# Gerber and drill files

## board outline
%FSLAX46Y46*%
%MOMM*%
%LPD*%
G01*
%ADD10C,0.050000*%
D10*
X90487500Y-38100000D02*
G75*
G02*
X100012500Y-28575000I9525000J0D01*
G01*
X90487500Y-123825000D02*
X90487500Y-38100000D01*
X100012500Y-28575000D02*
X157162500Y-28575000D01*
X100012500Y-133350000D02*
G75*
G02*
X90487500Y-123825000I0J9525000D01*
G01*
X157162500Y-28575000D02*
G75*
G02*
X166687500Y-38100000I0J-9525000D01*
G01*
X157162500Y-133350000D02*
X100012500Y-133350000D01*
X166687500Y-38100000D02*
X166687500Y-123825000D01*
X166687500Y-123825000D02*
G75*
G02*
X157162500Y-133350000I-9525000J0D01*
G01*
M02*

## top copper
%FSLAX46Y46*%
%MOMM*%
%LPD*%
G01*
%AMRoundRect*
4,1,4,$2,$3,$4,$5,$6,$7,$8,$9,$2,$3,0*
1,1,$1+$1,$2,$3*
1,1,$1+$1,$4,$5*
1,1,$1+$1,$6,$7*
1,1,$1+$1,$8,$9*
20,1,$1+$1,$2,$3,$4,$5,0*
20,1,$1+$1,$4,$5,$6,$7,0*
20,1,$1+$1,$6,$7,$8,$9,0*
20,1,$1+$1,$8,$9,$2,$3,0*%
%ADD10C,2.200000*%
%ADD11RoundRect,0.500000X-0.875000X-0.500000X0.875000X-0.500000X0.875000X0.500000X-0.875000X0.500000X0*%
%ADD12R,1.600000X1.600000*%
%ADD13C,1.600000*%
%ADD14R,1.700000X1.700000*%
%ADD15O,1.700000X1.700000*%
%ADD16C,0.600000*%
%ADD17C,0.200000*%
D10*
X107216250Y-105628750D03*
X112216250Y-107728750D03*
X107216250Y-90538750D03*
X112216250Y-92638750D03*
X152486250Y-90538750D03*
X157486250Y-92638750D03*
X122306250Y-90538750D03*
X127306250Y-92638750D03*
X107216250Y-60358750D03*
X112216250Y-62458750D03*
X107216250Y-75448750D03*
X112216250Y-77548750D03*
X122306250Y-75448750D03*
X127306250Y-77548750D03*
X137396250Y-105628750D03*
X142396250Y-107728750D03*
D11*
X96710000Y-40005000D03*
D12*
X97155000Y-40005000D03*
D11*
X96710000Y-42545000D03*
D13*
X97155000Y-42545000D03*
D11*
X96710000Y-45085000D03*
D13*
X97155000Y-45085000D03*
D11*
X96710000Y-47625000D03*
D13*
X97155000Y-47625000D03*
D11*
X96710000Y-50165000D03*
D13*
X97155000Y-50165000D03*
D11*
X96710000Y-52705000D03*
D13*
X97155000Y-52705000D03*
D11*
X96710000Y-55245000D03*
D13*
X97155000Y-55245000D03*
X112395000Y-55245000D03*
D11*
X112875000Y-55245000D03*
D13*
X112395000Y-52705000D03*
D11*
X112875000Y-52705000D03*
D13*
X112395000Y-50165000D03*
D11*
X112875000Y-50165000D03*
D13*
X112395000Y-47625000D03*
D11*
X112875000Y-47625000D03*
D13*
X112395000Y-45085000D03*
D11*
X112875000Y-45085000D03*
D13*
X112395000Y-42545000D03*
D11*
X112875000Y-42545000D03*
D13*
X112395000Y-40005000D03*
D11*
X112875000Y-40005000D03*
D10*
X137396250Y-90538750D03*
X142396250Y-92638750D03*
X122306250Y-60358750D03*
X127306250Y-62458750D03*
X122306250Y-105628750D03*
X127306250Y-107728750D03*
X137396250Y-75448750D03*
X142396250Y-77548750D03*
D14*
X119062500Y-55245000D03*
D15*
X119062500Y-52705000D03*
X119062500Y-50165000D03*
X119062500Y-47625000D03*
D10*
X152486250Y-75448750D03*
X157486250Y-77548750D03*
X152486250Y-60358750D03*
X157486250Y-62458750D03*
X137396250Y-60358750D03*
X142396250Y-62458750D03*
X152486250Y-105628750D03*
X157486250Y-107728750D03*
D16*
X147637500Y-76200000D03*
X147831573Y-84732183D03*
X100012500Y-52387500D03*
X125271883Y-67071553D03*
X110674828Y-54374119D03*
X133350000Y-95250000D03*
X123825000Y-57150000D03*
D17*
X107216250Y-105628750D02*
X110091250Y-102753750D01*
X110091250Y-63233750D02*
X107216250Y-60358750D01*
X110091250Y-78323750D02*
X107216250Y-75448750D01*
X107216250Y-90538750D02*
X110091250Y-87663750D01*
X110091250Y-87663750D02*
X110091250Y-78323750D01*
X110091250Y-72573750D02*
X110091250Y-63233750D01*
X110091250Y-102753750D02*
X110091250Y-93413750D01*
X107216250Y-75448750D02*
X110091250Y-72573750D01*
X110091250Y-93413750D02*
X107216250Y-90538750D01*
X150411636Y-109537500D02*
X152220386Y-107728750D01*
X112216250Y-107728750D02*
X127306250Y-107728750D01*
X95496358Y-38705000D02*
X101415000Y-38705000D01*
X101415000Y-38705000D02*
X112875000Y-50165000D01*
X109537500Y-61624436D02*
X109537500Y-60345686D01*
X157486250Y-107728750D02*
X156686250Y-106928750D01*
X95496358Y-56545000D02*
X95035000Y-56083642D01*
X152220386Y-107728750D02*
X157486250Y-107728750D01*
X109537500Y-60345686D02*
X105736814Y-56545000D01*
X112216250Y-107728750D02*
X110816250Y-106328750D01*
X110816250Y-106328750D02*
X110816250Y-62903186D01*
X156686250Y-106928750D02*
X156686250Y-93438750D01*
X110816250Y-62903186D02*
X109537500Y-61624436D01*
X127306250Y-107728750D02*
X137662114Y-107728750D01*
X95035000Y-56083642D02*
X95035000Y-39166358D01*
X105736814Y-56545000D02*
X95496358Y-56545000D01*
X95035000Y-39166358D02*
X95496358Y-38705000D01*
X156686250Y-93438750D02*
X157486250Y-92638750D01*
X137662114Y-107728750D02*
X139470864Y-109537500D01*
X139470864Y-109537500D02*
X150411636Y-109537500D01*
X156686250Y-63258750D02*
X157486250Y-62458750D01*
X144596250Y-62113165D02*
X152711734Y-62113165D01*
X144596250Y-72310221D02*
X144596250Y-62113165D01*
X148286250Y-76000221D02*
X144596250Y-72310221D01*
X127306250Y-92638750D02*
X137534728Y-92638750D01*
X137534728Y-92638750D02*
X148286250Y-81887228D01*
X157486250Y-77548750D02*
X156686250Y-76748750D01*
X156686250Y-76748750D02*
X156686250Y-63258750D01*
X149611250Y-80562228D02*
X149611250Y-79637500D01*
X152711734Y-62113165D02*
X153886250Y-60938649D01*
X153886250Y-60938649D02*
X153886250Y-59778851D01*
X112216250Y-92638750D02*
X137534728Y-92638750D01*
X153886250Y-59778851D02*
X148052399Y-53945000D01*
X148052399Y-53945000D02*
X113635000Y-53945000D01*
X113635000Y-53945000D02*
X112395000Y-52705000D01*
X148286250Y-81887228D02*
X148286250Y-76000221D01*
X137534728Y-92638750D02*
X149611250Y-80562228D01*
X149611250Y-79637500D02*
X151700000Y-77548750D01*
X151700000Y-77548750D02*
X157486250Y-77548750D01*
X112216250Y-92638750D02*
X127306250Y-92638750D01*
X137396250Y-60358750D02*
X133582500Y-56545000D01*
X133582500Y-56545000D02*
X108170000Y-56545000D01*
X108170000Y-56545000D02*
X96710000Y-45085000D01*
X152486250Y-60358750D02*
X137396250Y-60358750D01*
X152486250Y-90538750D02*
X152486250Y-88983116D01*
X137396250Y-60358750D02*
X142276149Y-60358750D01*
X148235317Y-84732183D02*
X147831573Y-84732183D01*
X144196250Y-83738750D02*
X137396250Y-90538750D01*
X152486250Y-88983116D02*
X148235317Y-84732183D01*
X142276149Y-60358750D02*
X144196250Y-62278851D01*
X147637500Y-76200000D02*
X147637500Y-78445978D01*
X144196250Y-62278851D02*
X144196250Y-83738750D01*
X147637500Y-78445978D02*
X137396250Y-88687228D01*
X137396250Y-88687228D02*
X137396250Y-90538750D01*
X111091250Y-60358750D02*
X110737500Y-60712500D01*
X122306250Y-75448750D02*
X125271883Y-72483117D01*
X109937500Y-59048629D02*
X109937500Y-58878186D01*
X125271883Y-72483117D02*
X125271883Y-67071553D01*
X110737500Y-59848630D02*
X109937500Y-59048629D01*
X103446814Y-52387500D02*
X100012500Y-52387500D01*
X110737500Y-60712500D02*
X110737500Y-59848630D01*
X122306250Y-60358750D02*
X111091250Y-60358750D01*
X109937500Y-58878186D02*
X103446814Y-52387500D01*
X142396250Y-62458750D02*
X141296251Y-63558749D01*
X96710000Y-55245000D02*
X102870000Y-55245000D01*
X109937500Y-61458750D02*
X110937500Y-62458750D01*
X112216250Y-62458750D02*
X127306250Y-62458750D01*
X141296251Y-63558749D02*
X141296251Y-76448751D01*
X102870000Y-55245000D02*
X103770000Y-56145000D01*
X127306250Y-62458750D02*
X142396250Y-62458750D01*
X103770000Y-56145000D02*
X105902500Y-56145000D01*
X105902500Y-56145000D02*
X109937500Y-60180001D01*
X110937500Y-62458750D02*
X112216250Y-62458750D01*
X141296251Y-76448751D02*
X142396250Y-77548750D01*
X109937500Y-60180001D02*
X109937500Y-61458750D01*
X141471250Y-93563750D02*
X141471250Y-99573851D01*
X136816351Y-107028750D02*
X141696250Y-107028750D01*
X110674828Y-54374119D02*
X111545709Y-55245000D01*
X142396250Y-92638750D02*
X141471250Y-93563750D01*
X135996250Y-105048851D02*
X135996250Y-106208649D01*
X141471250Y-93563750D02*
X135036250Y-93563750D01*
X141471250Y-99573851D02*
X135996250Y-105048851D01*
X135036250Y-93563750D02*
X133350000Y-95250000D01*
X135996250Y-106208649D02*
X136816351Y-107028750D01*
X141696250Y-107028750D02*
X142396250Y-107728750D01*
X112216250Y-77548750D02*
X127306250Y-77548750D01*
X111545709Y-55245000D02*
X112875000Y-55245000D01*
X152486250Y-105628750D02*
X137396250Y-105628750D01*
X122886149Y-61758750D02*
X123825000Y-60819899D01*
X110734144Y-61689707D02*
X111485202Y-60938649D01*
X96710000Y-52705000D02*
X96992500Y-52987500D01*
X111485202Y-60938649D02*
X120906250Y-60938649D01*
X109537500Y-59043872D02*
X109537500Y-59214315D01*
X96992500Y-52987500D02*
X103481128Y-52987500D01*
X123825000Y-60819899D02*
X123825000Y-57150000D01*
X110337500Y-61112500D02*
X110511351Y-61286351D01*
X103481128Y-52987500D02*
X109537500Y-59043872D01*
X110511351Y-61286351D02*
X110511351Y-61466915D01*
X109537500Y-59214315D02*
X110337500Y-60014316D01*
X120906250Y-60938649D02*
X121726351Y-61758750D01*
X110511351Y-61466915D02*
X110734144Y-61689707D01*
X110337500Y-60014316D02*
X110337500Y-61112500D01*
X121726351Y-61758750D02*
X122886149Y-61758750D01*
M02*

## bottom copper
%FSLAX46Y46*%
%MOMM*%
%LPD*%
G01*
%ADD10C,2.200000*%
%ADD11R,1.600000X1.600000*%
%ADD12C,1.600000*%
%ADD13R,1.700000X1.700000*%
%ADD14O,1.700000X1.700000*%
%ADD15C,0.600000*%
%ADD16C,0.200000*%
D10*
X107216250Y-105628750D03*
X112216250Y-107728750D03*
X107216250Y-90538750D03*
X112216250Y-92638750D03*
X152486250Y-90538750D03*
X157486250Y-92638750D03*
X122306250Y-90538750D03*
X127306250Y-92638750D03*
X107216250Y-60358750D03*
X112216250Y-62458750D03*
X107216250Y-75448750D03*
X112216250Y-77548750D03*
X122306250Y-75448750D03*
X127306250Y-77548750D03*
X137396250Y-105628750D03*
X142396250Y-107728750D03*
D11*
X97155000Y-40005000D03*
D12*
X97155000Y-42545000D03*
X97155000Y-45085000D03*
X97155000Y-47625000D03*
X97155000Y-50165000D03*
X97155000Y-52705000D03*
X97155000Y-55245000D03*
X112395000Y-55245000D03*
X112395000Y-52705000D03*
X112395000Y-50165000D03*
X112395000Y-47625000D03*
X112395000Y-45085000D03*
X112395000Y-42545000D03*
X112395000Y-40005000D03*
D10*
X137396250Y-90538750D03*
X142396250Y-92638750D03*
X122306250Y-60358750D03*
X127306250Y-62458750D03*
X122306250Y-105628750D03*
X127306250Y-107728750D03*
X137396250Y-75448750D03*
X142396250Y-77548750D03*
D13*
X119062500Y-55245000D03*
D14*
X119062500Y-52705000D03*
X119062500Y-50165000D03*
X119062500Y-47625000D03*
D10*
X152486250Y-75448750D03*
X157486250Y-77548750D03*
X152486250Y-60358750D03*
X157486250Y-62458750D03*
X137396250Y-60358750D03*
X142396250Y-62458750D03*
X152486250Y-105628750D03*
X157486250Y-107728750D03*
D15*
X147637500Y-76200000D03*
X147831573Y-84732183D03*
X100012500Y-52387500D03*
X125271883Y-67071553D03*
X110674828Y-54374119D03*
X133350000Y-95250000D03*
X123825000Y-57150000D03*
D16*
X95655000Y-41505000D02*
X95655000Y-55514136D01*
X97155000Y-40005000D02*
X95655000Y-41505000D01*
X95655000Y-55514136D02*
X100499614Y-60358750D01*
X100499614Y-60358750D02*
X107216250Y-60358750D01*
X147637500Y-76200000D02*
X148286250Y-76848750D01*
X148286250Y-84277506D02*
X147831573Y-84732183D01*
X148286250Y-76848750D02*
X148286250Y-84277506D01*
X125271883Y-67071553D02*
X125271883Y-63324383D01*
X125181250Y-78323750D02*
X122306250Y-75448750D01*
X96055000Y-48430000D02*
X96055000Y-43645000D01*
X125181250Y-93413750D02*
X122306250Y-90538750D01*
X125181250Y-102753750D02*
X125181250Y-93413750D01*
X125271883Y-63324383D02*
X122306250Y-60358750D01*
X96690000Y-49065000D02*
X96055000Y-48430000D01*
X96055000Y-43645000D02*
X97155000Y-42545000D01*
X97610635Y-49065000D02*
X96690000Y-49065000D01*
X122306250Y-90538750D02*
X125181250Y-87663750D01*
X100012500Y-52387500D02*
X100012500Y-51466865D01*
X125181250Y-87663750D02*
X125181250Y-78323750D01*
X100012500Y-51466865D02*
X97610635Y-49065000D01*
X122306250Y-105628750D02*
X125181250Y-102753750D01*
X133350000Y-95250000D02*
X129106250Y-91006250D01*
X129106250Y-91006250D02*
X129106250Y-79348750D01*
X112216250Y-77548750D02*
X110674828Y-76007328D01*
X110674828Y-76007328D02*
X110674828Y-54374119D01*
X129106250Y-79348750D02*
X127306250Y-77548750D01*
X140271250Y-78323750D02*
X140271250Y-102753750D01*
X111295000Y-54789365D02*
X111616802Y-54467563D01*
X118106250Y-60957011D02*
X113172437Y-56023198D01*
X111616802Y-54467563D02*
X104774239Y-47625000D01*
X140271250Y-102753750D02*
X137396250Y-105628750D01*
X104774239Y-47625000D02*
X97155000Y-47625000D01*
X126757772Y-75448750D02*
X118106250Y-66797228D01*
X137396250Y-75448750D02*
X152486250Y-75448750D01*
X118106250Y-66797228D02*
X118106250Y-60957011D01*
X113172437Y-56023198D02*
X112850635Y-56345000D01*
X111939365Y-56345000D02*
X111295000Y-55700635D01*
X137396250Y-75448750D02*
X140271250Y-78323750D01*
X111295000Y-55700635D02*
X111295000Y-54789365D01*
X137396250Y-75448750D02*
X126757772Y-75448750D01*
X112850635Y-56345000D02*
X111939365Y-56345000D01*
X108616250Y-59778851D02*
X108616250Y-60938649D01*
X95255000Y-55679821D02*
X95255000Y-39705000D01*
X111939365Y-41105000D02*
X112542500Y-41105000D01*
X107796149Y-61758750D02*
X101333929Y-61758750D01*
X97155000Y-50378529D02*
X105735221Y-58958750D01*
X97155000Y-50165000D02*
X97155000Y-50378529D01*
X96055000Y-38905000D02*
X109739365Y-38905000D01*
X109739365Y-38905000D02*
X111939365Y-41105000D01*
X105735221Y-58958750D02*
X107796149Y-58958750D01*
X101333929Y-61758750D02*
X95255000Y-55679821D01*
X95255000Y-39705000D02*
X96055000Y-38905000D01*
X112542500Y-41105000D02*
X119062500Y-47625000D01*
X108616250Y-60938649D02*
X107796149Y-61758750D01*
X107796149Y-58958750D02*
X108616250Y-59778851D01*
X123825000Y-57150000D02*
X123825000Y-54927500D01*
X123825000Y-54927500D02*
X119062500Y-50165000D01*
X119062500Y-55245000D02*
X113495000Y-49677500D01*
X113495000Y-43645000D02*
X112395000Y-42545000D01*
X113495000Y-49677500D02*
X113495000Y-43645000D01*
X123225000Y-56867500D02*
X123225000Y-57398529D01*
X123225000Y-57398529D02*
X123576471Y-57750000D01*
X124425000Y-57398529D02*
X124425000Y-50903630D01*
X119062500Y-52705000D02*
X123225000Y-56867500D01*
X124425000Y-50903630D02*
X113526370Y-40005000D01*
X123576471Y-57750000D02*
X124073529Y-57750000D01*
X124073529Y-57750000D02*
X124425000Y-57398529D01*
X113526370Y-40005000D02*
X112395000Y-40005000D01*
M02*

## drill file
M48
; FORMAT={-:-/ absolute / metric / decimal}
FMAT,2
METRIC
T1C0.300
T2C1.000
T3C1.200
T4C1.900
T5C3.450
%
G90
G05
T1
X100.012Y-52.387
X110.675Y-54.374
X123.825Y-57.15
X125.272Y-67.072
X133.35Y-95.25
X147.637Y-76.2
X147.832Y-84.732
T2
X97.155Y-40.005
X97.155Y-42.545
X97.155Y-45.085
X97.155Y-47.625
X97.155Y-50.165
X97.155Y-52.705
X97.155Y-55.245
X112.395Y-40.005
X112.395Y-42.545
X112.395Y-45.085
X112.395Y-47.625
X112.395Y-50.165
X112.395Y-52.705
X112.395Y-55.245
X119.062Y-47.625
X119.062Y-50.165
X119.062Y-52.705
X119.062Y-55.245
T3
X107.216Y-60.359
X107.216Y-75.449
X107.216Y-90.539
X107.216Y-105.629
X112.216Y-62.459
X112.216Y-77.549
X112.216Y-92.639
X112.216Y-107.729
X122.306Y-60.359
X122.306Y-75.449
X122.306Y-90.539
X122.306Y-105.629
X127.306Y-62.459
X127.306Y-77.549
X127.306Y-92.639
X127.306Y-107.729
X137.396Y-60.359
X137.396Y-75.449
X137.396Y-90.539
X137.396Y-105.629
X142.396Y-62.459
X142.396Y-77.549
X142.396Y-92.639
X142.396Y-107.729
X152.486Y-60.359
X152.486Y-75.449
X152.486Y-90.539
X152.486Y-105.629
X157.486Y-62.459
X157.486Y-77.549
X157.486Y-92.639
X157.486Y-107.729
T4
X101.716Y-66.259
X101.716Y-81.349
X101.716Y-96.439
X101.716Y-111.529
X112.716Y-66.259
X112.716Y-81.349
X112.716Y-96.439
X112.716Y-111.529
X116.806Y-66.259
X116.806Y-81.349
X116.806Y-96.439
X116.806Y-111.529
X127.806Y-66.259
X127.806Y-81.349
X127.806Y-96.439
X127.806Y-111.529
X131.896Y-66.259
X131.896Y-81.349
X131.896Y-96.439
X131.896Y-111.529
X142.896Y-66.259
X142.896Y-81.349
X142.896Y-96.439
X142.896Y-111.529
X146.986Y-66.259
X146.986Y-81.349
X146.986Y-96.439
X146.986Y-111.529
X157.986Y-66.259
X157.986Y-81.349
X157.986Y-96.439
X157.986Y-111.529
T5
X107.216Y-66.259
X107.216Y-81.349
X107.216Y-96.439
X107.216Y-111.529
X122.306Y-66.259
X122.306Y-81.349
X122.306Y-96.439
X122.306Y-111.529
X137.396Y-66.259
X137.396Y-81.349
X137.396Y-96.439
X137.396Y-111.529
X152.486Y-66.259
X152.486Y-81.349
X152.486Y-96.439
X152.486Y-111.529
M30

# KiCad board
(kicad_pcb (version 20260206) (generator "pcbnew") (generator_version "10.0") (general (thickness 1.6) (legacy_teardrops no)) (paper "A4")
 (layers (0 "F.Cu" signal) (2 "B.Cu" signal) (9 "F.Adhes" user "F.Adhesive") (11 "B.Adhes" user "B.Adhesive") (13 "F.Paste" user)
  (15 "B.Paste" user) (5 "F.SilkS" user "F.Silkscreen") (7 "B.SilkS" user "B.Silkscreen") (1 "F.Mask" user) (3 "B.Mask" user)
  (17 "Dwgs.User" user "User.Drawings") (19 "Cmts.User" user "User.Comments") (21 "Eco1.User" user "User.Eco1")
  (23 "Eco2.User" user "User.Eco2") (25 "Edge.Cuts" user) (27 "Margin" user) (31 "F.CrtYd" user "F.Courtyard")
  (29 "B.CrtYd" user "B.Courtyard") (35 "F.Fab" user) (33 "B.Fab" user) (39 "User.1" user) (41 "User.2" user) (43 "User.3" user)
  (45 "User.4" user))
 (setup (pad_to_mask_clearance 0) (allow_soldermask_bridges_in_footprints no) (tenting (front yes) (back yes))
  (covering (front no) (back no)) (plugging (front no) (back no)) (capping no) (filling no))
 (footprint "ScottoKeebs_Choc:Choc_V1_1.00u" (layer "F.Cu") (at 107.21625 111.52875)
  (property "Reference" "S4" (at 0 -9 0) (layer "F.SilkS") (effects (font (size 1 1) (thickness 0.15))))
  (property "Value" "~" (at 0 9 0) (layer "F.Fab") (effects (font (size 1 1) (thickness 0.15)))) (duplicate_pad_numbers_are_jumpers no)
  (pad "" np_thru_hole circle (at -5.5 0) (size 1.9 1.9) (drill 1.9) (layers "*.Cu" "*.Mask"))
  (pad "" np_thru_hole circle (at 0 0) (size 3.45 3.45) (drill 3.45) (layers "*.Cu" "*.Mask"))
  (pad "" np_thru_hole circle (at 5.5 0) (size 1.9 1.9) (drill 1.9) (layers "*.Cu" "*.Mask"))
  (pad "1" thru_hole circle (at 0 -5.9) (size 2.2 2.2) (drill 1.2) (layers "*.Cu" "*.Mask") (remove_unused_layers no) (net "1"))
  (pad "2" thru_hole circle (at 5 -3.8) (size 2.2 2.2) (drill 1.2) (layers "*.Cu" "*.Mask") (remove_unused_layers no) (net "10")))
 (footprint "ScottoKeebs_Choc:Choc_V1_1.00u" (layer "F.Cu") (at 107.21625 96.43875)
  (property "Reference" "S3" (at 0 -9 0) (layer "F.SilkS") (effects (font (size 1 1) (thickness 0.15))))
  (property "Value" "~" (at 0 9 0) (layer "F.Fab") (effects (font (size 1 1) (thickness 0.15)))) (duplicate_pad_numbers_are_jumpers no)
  (pad "" np_thru_hole circle (at -5.5 0) (size 1.9 1.9) (drill 1.9) (layers "*.Cu" "*.Mask"))
  (pad "" np_thru_hole circle (at 0 0) (size 3.45 3.45) (drill 3.45) (layers "*.Cu" "*.Mask"))
  (pad "" np_thru_hole circle (at 5.5 0) (size 1.9 1.9) (drill 1.9) (layers "*.Cu" "*.Mask"))
  (pad "1" thru_hole circle (at 0 -5.9) (size 2.2 2.2) (drill 1.2) (layers "*.Cu" "*.Mask") (remove_unused_layers no) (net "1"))
  (pad "2" thru_hole circle (at 5 -3.8) (size 2.2 2.2) (drill 1.2) (layers "*.Cu" "*.Mask") (remove_unused_layers no) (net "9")))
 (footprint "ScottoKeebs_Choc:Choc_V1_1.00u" (layer "F.Cu") (at 152.48625 96.43875)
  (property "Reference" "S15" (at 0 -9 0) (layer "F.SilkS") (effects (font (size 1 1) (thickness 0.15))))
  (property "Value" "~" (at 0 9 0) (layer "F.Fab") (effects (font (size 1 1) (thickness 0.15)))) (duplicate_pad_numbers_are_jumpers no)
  (pad "" np_thru_hole circle (at -5.5 0) (size 1.9 1.9) (drill 1.9) (layers "*.Cu" "*.Mask"))
  (pad "" np_thru_hole circle (at 0 0) (size 3.45 3.45) (drill 3.45) (layers "*.Cu" "*.Mask"))
  (pad "" np_thru_hole circle (at 5.5 0) (size 1.9 1.9) (drill 1.9) (layers "*.Cu" "*.Mask"))
  (pad "1" thru_hole circle (at 0 -5.9) (size 2.2 2.2) (drill 1.2) (layers "*.Cu" "*.Mask") (remove_unused_layers no) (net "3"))
  (pad "2" thru_hole circle (at 5 -3.8) (size 2.2 2.2) (drill 1.2) (layers "*.Cu" "*.Mask") (remove_unused_layers no) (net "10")))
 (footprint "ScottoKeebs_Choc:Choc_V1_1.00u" (layer "F.Cu") (at 122.30625 96.43875)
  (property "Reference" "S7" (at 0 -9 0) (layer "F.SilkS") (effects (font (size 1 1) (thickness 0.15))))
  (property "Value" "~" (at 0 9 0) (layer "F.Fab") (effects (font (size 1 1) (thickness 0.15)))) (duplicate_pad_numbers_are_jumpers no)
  (pad "" np_thru_hole circle (at -5.5 0) (size 1.9 1.9) (drill 1.9) (layers "*.Cu" "*.Mask"))
  (pad "" np_thru_hole circle (at 0 0) (size 3.45 3.45) (drill 3.45) (layers "*.Cu" "*.Mask"))
  (pad "" np_thru_hole circle (at 5.5 0) (size 1.9 1.9) (drill 1.9) (layers "*.Cu" "*.Mask"))
  (pad "1" thru_hole circle (at 0 -5.9) (size 2.2 2.2) (drill 1.2) (layers "*.Cu" "*.Mask") (remove_unused_layers no) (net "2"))
  (pad "2" thru_hole circle (at 5 -3.8) (size 2.2 2.2) (drill 1.2) (layers "*.Cu" "*.Mask") (remove_unused_layers no) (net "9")))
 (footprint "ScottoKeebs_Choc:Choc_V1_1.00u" (layer "F.Cu") (at 107.21625 66.25875)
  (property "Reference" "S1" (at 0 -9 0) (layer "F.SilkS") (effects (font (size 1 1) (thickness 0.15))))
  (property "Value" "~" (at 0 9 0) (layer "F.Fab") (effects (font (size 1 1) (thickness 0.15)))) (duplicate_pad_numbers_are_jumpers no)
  (pad "" np_thru_hole circle (at -5.5 0) (size 1.9 1.9) (drill 1.9) (layers "*.Cu" "*.Mask"))
  (pad "" np_thru_hole circle (at 0 0) (size 3.45 3.45) (drill 3.45) (layers "*.Cu" "*.Mask"))
  (pad "" np_thru_hole circle (at 5.5 0) (size 1.9 1.9) (drill 1.9) (layers "*.Cu" "*.Mask"))
  (pad "1" thru_hole circle (at 0 -5.9) (size 2.2 2.2) (drill 1.2) (layers "*.Cu" "*.Mask") (remove_unused_layers no) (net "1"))
  (pad "2" thru_hole circle (at 5 -3.8) (size 2.2 2.2) (drill 1.2) (layers "*.Cu" "*.Mask") (remove_unused_layers no) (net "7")))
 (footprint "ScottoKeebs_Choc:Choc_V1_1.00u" (layer "F.Cu") (at 107.21625 81.34875)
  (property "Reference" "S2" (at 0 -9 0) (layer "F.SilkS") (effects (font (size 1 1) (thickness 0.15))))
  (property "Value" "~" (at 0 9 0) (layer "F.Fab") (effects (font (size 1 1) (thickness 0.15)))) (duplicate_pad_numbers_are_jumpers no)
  (pad "" np_thru_hole circle (at -5.5 0) (size 1.9 1.9) (drill 1.9) (layers "*.Cu" "*.Mask"))
  (pad "" np_thru_hole circle (at 0 0) (size 3.45 3.45) (drill 3.45) (layers "*.Cu" "*.Mask"))
  (pad "" np_thru_hole circle (at 5.5 0) (size 1.9 1.9) (drill 1.9) (layers "*.Cu" "*.Mask"))
  (pad "1" thru_hole circle (at 0 -5.9) (size 2.2 2.2) (drill 1.2) (layers "*.Cu" "*.Mask") (remove_unused_layers no) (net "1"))
  (pad "2" thru_hole circle (at 5 -3.8) (size 2.2 2.2) (drill 1.2) (layers "*.Cu" "*.Mask") (remove_unused_layers no) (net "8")))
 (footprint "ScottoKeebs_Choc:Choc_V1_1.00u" (layer "F.Cu") (at 122.30625 81.34875)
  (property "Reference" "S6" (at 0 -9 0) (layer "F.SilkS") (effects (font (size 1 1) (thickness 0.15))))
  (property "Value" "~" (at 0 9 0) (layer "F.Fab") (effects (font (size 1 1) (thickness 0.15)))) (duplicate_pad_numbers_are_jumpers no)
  (pad "" np_thru_hole circle (at -5.5 0) (size 1.9 1.9) (drill 1.9) (layers "*.Cu" "*.Mask"))
  (pad "" np_thru_hole circle (at 0 0) (size 3.45 3.45) (drill 3.45) (layers "*.Cu" "*.Mask"))
  (pad "" np_thru_hole circle (at 5.5 0) (size 1.9 1.9) (drill 1.9) (layers "*.Cu" "*.Mask"))
  (pad "1" thru_hole circle (at 0 -5.9) (size 2.2 2.2) (drill 1.2) (layers "*.Cu" "*.Mask") (remove_unused_layers no) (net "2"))
  (pad "2" thru_hole circle (at 5 -3.8) (size 2.2 2.2) (drill 1.2) (layers "*.Cu" "*.Mask") (remove_unused_layers no) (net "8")))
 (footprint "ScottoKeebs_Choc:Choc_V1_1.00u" (layer "F.Cu") (at 137.39625 111.52875)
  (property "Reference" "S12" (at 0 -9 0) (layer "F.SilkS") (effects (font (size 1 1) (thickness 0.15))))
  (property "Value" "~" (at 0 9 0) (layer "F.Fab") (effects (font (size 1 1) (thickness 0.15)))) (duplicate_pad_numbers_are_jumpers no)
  (pad "" np_thru_hole circle (at -5.5 0) (size 1.9 1.9) (drill 1.9) (layers "*.Cu" "*.Mask"))
  (pad "" np_thru_hole circle (at 0 0) (size 3.45 3.45) (drill 3.45) (layers "*.Cu" "*.Mask"))
  (pad "" np_thru_hole circle (at 5.5 0) (size 1.9 1.9) (drill 1.9) (layers "*.Cu" "*.Mask"))
  (pad "1" thru_hole circle (at 0 -5.9) (size 2.2 2.2) (drill 1.2) (layers "*.Cu" "*.Mask") (remove_unused_layers no) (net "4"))
  (pad "2" thru_hole circle (at 5 -3.8) (size 2.2 2.2) (drill 1.2) (layers "*.Cu" "*.Mask") (remove_unused_layers no) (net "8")))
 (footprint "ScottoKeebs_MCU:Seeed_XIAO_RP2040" (layer "F.Cu") (at 104.775 47.625)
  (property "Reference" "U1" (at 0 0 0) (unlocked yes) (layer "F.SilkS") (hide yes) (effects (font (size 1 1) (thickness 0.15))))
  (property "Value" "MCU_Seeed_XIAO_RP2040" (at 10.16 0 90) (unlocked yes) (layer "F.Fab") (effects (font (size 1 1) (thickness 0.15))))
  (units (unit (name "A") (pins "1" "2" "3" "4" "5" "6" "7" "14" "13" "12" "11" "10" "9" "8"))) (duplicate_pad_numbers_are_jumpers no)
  (pad "1" smd roundrect (at -8.065 -7.62) (size 2.75 2) (layers "F.Cu" "F.Mask" "F.Paste") (roundrect_rratio 0.25) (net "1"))
  (pad "1" thru_hole rect (at -7.62 -7.62 90) (size 1.6 1.6) (drill 1) (layers "*.Cu" "*.Mask") (remove_unused_layers no) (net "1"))
  (pad "2" smd roundrect (at -8.065 -5.08) (size 2.75 2) (layers "F.Cu" "F.Mask" "F.Paste") (roundrect_rratio 0.25) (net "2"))
  (pad "2" thru_hole circle (at -7.62 -5.08 90) (size 1.6 1.6) (drill 1) (layers "*.Cu" "*.Mask") (remove_unused_layers no) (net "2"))
  (pad "3" smd roundrect (at -8.065 -2.54) (size 2.75 2) (layers "F.Cu" "F.Mask" "F.Paste") (roundrect_rratio 0.25) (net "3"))
  (pad "3" thru_hole circle (at -7.62 -2.54 90) (size 1.6 1.6) (drill 1) (layers "*.Cu" "*.Mask") (remove_unused_layers no) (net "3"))
  (pad "4" smd roundrect (at -8.065 0) (size 2.75 2) (layers "F.Cu" "F.Mask" "F.Paste") (roundrect_rratio 0.25) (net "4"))
  (pad "4" thru_hole circle (at -7.62 0 90) (size 1.6 1.6) (drill 1) (layers "*.Cu" "*.Mask") (remove_unused_layers no) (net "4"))
  (pad "5" smd roundrect (at -8.065 2.54) (size 2.75 2) (layers "F.Cu" "F.Mask" "F.Paste") (roundrect_rratio 0.25) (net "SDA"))
  (pad "5" thru_hole circle (at -7.62 2.54 90) (size 1.6 1.6) (drill 1) (layers "*.Cu" "*.Mask") (remove_unused_layers no) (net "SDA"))
  (pad "6" smd roundrect (at -8.065 5.08) (size 2.75 2) (layers "F.Cu" "F.Mask" "F.Paste") (roundrect_rratio 0.25) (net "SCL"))
  (pad "6" thru_hole circle (at -7.62 5.08 90) (size 1.6 1.6) (drill 1) (layers "*.Cu" "*.Mask") (remove_unused_layers no) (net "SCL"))
  (pad "7" smd roundrect (at -8.065 7.62) (size 2.75 2) (layers "F.Cu" "F.Mask" "F.Paste") (roundrect_rratio 0.25) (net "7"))
  (pad "7" thru_hole circle (at -7.62 7.62 90) (size 1.6 1.6) (drill 1) (layers "*.Cu" "*.Mask") (remove_unused_layers no) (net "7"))
  (pad "8" thru_hole circle (at 7.62 7.62 90) (size 1.6 1.6) (drill 1) (layers "*.Cu" "*.Mask") (remove_unused_layers no) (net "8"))
  (pad "8" smd roundrect (at 8.1 7.62) (size 2.75 2) (layers "F.Cu" "F.Mask" "F.Paste") (roundrect_rratio 0.25) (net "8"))
  (pad "9" thru_hole circle (at 7.62 5.08 90) (size 1.6 1.6) (drill 1) (layers "*.Cu" "*.Mask") (remove_unused_layers no) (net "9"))
  (pad "9" smd roundrect (at 8.1 5.08) (size 2.75 2) (layers "F.Cu" "F.Mask" "F.Paste") (roundrect_rratio 0.25) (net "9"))
  (pad "10" thru_hole circle (at 7.62 2.54 90) (size 1.6 1.6) (drill 1) (layers "*.Cu" "*.Mask") (remove_unused_layers no) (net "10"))
  (pad "10" smd roundrect (at 8.1 2.54) (size 2.75 2) (layers "F.Cu" "F.Mask" "F.Paste") (roundrect_rratio 0.25) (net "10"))
  (pad "11" thru_hole circle (at 7.62 0 90) (size 1.6 1.6) (drill 1) (layers "*.Cu" "*.Mask") (remove_unused_layers no) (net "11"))
  (pad "11" smd roundrect (at 8.1 0) (size 2.75 2) (layers "F.Cu" "F.Mask" "F.Paste") (roundrect_rratio 0.25) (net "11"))
  (pad "12" thru_hole circle (at 7.62 -2.54 90) (size 1.6 1.6) (drill 1) (layers "*.Cu" "*.Mask") (remove_unused_layers no) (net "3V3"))
  (pad "12" smd roundrect (at 8.1 -2.54) (size 2.75 2) (layers "F.Cu" "F.Mask" "F.Paste") (roundrect_rratio 0.25) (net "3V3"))
  (pad "13" thru_hole circle (at 7.62 -5.08 90) (size 1.6 1.6) (drill 1) (layers "*.Cu" "*.Mask") (remove_unused_layers no) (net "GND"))
  (pad "13" smd roundrect (at 8.1 -5.08) (size 2.75 2) (layers "F.Cu" "F.Mask" "F.Paste") (roundrect_rratio 0.25) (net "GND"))
  (pad "14" thru_hole circle (at 7.62 -7.62 90) (size 1.6 1.6) (drill 1) (layers "*.Cu" "*.Mask") (remove_unused_layers no) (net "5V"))
  (pad "14" smd roundrect (at 8.1 -7.62) (size 2.75 2) (layers "F.Cu" "F.Mask" "F.Paste") (roundrect_rratio 0.25) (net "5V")))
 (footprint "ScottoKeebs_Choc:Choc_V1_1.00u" (layer "F.Cu") (at 137.39625 96.43875)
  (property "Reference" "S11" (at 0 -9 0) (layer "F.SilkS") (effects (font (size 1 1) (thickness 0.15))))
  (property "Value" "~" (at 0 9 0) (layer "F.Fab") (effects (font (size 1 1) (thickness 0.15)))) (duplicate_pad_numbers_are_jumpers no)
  (pad "" np_thru_hole circle (at -5.5 0) (size 1.9 1.9) (drill 1.9) (layers "*.Cu" "*.Mask"))
  (pad "" np_thru_hole circle (at 0 0) (size 3.45 3.45) (drill 3.45) (layers "*.Cu" "*.Mask"))
  (pad "" np_thru_hole circle (at 5.5 0) (size 1.9 1.9) (drill 1.9) (layers "*.Cu" "*.Mask"))
  (pad "1" thru_hole circle (at 0 -5.9) (size 2.2 2.2) (drill 1.2) (layers "*.Cu" "*.Mask") (remove_unused_layers no) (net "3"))
  (pad "2" thru_hole circle (at 5 -3.8) (size 2.2 2.2) (drill 1.2) (layers "*.Cu" "*.Mask") (remove_unused_layers no) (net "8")))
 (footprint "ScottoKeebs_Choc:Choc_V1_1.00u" (layer "F.Cu") (at 122.30625 66.25875)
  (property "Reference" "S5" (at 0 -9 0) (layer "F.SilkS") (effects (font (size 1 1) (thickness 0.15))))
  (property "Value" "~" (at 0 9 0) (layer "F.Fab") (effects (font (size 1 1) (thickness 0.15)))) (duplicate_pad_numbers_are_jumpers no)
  (pad "" np_thru_hole circle (at -5.5 0) (size 1.9 1.9) (drill 1.9) (layers "*.Cu" "*.Mask"))
  (pad "" np_thru_hole circle (at 0 0) (size 3.45 3.45) (drill 3.45) (layers "*.Cu" "*.Mask"))
  (pad "" np_thru_hole circle (at 5.5 0) (size 1.9 1.9) (drill 1.9) (layers "*.Cu" "*.Mask"))
  (pad "1" thru_hole circle (at 0 -5.9) (size 2.2 2.2) (drill 1.2) (layers "*.Cu" "*.Mask") (remove_unused_layers no) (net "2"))
  (pad "2" thru_hole circle (at 5 -3.8) (size 2.2 2.2) (drill 1.2) (layers "*.Cu" "*.Mask") (remove_unused_layers no) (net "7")))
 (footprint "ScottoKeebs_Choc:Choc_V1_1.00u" (layer "F.Cu") (at 122.30625 111.52875)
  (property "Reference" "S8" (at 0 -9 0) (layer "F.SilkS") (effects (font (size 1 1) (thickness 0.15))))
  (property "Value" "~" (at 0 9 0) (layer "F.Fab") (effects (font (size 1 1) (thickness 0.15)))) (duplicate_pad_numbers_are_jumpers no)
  (pad "" np_thru_hole circle (at -5.5 0) (size 1.9 1.9) (drill 1.9) (layers "*.Cu" "*.Mask"))
  (pad "" np_thru_hole circle (at 0 0) (size 3.45 3.45) (drill 3.45) (layers "*.Cu" "*.Mask"))
  (pad "" np_thru_hole circle (at 5.5 0) (size 1.9 1.9) (drill 1.9) (layers "*.Cu" "*.Mask"))
  (pad "1" thru_hole circle (at 0 -5.9) (size 2.2 2.2) (drill 1.2) (layers "*.Cu" "*.Mask") (remove_unused_layers no) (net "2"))
  (pad "2" thru_hole circle (at 5 -3.8) (size 2.2 2.2) (drill 1.2) (layers "*.Cu" "*.Mask") (remove_unused_layers no) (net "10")))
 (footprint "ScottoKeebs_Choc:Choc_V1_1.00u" (layer "F.Cu") (at 137.39625 81.34875)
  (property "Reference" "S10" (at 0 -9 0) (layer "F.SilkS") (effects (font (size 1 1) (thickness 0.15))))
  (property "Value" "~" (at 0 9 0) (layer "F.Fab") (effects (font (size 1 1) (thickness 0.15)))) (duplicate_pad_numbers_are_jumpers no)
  (pad "" np_thru_hole circle (at -5.5 0) (size 1.9 1.9) (drill 1.9) (layers "*.Cu" "*.Mask"))
  (pad "" np_thru_hole circle (at 0 0) (size 3.45 3.45) (drill 3.45) (layers "*.Cu" "*.Mask"))
  (pad "" np_thru_hole circle (at 5.5 0) (size 1.9 1.9) (drill 1.9) (layers "*.Cu" "*.Mask"))
  (pad "1" thru_hole circle (at 0 -5.9) (size 2.2 2.2) (drill 1.2) (layers "*.Cu" "*.Mask") (remove_unused_layers no) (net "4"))
  (pad "2" thru_hole circle (at 5 -3.8) (size 2.2 2.2) (drill 1.2) (layers "*.Cu" "*.Mask") (remove_unused_layers no) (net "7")))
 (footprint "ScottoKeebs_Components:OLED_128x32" (layer "F.Cu") (at 117.4625 45.445)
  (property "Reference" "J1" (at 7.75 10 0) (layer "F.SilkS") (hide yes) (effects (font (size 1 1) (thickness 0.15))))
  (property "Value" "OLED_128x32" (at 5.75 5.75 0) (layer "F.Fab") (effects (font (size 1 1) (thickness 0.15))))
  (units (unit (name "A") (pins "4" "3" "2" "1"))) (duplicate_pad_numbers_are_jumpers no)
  (pad "1" thru_hole rect (at 1.6 9.8 180) (size 1.7 1.7) (drill 1) (layers "*.Cu" "*.Mask") (remove_unused_layers no) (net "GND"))
  (pad "2" thru_hole oval (at 1.6 7.26 180) (size 1.7 1.7) (drill 1) (layers "*.Cu" "*.Mask") (remove_unused_layers no) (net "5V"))
  (pad "3" thru_hole oval (at 1.6 4.72 180) (size 1.7 1.7) (drill 1) (layers "*.Cu" "*.Mask") (remove_unused_layers no) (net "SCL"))
  (pad "4" thru_hole oval (at 1.6 2.18 180) (size 1.7 1.7) (drill 1) (layers "*.Cu" "*.Mask") (remove_unused_layers no) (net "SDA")))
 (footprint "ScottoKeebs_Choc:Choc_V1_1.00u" (layer "F.Cu") (at 152.48625 81.34875)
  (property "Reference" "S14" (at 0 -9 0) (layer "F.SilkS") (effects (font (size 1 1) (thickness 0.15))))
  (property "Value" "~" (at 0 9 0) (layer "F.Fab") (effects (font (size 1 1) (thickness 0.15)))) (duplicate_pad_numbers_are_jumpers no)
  (pad "" np_thru_hole circle (at -5.5 0) (size 1.9 1.9) (drill 1.9) (layers "*.Cu" "*.Mask"))
  (pad "" np_thru_hole circle (at 0 0) (size 3.45 3.45) (drill 3.45) (layers "*.Cu" "*.Mask"))
  (pad "" np_thru_hole circle (at 5.5 0) (size 1.9 1.9) (drill 1.9) (layers "*.Cu" "*.Mask"))
  (pad "1" thru_hole circle (at 0 -5.9) (size 2.2 2.2) (drill 1.2) (layers "*.Cu" "*.Mask") (remove_unused_layers no) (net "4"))
  (pad "2" thru_hole circle (at 5 -3.8) (size 2.2 2.2) (drill 1.2) (layers "*.Cu" "*.Mask") (remove_unused_layers no) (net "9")))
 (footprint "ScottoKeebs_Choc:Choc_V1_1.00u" (layer "F.Cu") (at 152.48625 66.25875)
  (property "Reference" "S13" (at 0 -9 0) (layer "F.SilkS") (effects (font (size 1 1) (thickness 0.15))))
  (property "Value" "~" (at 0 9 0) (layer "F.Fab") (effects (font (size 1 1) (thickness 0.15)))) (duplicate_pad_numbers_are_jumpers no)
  (pad "" np_thru_hole circle (at -5.5 0) (size 1.9 1.9) (drill 1.9) (layers "*.Cu" "*.Mask"))
  (pad "" np_thru_hole circle (at 0 0) (size 3.45 3.45) (drill 3.45) (layers "*.Cu" "*.Mask"))
  (pad "" np_thru_hole circle (at 5.5 0) (size 1.9 1.9) (drill 1.9) (layers "*.Cu" "*.Mask"))
  (pad "1" thru_hole circle (at 0 -5.9) (size 2.2 2.2) (drill 1.2) (layers "*.Cu" "*.Mask") (remove_unused_layers no) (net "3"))
  (pad "2" thru_hole circle (at 5 -3.8) (size 2.2 2.2) (drill 1.2) (layers "*.Cu" "*.Mask") (remove_unused_layers no) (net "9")))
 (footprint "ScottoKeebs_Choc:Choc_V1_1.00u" (layer "F.Cu") (at 137.39625 66.25875)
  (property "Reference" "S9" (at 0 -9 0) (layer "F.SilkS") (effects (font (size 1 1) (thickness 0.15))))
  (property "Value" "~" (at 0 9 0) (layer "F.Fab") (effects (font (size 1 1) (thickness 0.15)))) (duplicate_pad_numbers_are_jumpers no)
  (pad "" np_thru_hole circle (at -5.5 0) (size 1.9 1.9) (drill 1.9) (layers "*.Cu" "*.Mask"))
  (pad "" np_thru_hole circle (at 0 0) (size 3.45 3.45) (drill 3.45) (layers "*.Cu" "*.Mask"))
  (pad "" np_thru_hole circle (at 5.5 0) (size 1.9 1.9) (drill 1.9) (layers "*.Cu" "*.Mask"))
  (pad "1" thru_hole circle (at 0 -5.9) (size 2.2 2.2) (drill 1.2) (layers "*.Cu" "*.Mask") (remove_unused_layers no) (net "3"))
  (pad "2" thru_hole circle (at 5 -3.8) (size 2.2 2.2) (drill 1.2) (layers "*.Cu" "*.Mask") (remove_unused_layers no) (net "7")))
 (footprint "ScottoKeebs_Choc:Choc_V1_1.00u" (layer "F.Cu") (at 152.48625 111.52875)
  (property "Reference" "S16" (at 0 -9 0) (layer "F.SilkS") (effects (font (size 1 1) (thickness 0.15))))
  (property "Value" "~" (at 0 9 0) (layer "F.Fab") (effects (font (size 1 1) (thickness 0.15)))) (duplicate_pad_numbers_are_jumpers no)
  (pad "" np_thru_hole circle (at -5.5 0) (size 1.9 1.9) (drill 1.9) (layers "*.Cu" "*.Mask"))
  (pad "" np_thru_hole circle (at 0 0) (size 3.45 3.45) (drill 3.45) (layers "*.Cu" "*.Mask"))
  (pad "" np_thru_hole circle (at 5.5 0) (size 1.9 1.9) (drill 1.9) (layers "*.Cu" "*.Mask"))
  (pad "1" thru_hole circle (at 0 -5.9) (size 2.2 2.2) (drill 1.2) (layers "*.Cu" "*.Mask") (remove_unused_layers no) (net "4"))
  (pad "2" thru_hole circle (at 5 -3.8) (size 2.2 2.2) (drill 1.2) (layers "*.Cu" "*.Mask") (remove_unused_layers no) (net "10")))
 (gr_arc (start 90.4875 38.1) (mid 93.277308 31.364808) (end 100.0125 28.575) (stroke (width 0.05) (type default)) (layer "Edge.Cuts"))
 (gr_line (start 90.4875 123.825) (end 90.4875 38.1) (stroke (width 0.05) (type default)) (layer "Edge.Cuts"))
 (gr_line (start 100.0125 28.575) (end 157.1625 28.575) (stroke (width 0.05) (type default)) (layer "Edge.Cuts"))
 (gr_arc (start 100.0125 133.35) (mid 93.277308 130.560192) (end 90.4875 123.825) (stroke (width 0.05) (type default)) (layer "Edge.Cuts"))
 (gr_arc (start 157.1625 28.575) (mid 163.897692 31.364808) (end 166.6875 38.1) (stroke (width 0.05) (type default)) (layer "Edge.Cuts"))
 (gr_line (start 157.1625 133.35) (end 100.0125 133.35) (stroke (width 0.05) (type default)) (layer "Edge.Cuts"))
 (gr_line (start 166.6875 38.1) (end 166.6875 123.825) (stroke (width 0.05) (type default)) (layer "Edge.Cuts"))
 (gr_arc (start 166.6875 123.825) (mid 163.897692 130.560192) (end 157.1625 133.35) (stroke (width 0.05) (type default)) (layer "Edge.Cuts"))
 (segment (start 107.21625 105.62875) (end 110.09125 102.75375) (width 0.2) (layer "F.Cu") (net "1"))
 (segment (start 110.09125 63.23375) (end 107.21625 60.35875) (width 0.2) (layer "F.Cu") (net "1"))
 (segment (start 110.09125 78.32375) (end 107.21625 75.44875) (width 0.2) (layer "F.Cu") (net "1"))
 (segment (start 107.21625 90.53875) (end 110.09125 87.66375) (width 0.2) (layer "F.Cu") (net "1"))
 (segment (start 110.09125 87.66375) (end 110.09125 78.32375) (width 0.2) (layer "F.Cu") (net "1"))
 (segment (start 110.09125 72.57375) (end 110.09125 63.23375) (width 0.2) (layer "F.Cu") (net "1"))
 (segment (start 110.09125 102.75375) (end 110.09125 93.41375) (width 0.2) (layer "F.Cu") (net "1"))
 (segment (start 107.21625 75.44875) (end 110.09125 72.57375) (width 0.2) (layer "F.Cu") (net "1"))
 (segment (start 110.09125 93.41375) (end 107.21625 90.53875) (width 0.2) (layer "F.Cu") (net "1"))
 (segment (start 95.655 41.505) (end 95.655 55.514136) (width 0.2) (layer "B.Cu") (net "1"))
 (segment (start 97.155 40.005) (end 95.655 41.505) (width 0.2) (layer "B.Cu") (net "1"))
 (segment (start 95.655 55.514136) (end 100.499614 60.35875) (width 0.2) (layer "B.Cu") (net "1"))
 (segment (start 100.499614 60.35875) (end 107.21625 60.35875) (width 0.2) (layer "B.Cu") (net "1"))
 (segment (start 150.411636 109.5375) (end 152.220386 107.72875) (width 0.2) (layer "F.Cu") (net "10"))
 (segment (start 112.21625 107.72875) (end 127.30625 107.72875) (width 0.2) (layer "F.Cu") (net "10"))
 (segment (start 95.496358 38.705) (end 101.415 38.705) (width 0.2) (layer "F.Cu") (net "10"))
 (segment (start 101.415 38.705) (end 112.875 50.165) (width 0.2) (layer "F.Cu") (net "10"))
 (segment (start 109.5375 61.624436) (end 109.5375 60.345686) (width 0.2) (layer "F.Cu") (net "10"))
 (segment (start 157.48625 107.72875) (end 156.68625 106.92875) (width 0.2) (layer "F.Cu") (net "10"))
 (segment (start 95.496358 56.545) (end 95.035 56.083642) (width 0.2) (layer "F.Cu") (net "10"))
 (segment (start 152.220386 107.72875) (end 157.48625 107.72875) (width 0.2) (layer "F.Cu") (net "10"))
 (segment (start 109.5375 60.345686) (end 105.736814 56.545) (width 0.2) (layer "F.Cu") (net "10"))
 (segment (start 112.21625 107.72875) (end 110.81625 106.32875) (width 0.2) (layer "F.Cu") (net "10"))
 (segment (start 110.81625 106.32875) (end 110.81625 62.903186) (width 0.2) (layer "F.Cu") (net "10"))
 (segment (start 156.68625 106.92875) (end 156.68625 93.43875) (width 0.2) (layer "F.Cu") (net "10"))
 (segment (start 110.81625 62.903186) (end 109.5375 61.624436) (width 0.2) (layer "F.Cu") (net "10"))
 (segment (start 127.30625 107.72875) (end 137.662114 107.72875) (width 0.2) (layer "F.Cu") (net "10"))
 (segment (start 95.035 56.083642) (end 95.035 39.166358) (width 0.2) (layer "F.Cu") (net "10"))
 (segment (start 105.736814 56.545) (end 95.496358 56.545) (width 0.2) (layer "F.Cu") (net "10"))
 (segment (start 95.035 39.166358) (end 95.496358 38.705) (width 0.2) (layer "F.Cu") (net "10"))
 (segment (start 156.68625 93.43875) (end 157.48625 92.63875) (width 0.2) (layer "F.Cu") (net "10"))
 (segment (start 137.662114 107.72875) (end 139.470864 109.5375) (width 0.2) (layer "F.Cu") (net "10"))
 (segment (start 139.470864 109.5375) (end 150.411636 109.5375) (width 0.2) (layer "F.Cu") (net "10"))
 (segment (start 156.68625 63.25875) (end 157.48625 62.45875) (width 0.2) (layer "F.Cu") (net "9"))
 (segment (start 144.59625 62.113165) (end 152.711734 62.113165) (width 0.2) (layer "F.Cu") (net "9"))
 (segment (start 144.59625 72.310221) (end 144.59625 62.113165) (width 0.2) (layer "F.Cu") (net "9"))
 (segment (start 148.28625 76.000221) (end 144.59625 72.310221) (width 0.2) (layer "F.Cu") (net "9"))
 (segment (start 127.30625 92.63875) (end 137.534728 92.63875) (width 0.2) (layer "F.Cu") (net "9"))
 (segment (start 137.534728 92.63875) (end 148.28625 81.887228) (width 0.2) (layer "F.Cu") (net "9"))
 (segment (start 157.48625 77.54875) (end 156.68625 76.74875) (width 0.2) (layer "F.Cu") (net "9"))
 (segment (start 156.68625 76.74875) (end 156.68625 63.25875) (width 0.2) (layer "F.Cu") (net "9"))
 (segment (start 149.61125 80.562228) (end 149.61125 79.6375) (width 0.2) (layer "F.Cu") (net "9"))
 (segment (start 152.711734 62.113165) (end 153.88625 60.938649) (width 0.2) (layer "F.Cu") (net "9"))
 (segment (start 153.88625 60.938649) (end 153.88625 59.778851) (width 0.2) (layer "F.Cu") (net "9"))
 (segment (start 112.21625 92.63875) (end 137.534728 92.63875) (width 0.2) (layer "F.Cu") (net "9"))
 (segment (start 153.88625 59.778851) (end 148.052399 53.945) (width 0.2) (layer "F.Cu") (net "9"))
 (segment (start 148.052399 53.945) (end 113.635 53.945) (width 0.2) (layer "F.Cu") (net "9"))
 (segment (start 113.635 53.945) (end 112.395 52.705) (width 0.2) (layer "F.Cu") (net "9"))
 (segment (start 148.28625 81.887228) (end 148.28625 76.000221) (width 0.2) (layer "F.Cu") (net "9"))
 (segment (start 137.534728 92.63875) (end 149.61125 80.562228) (width 0.2) (layer "F.Cu") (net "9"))
 (segment (start 149.61125 79.6375) (end 151.7 77.54875) (width 0.2) (layer "F.Cu") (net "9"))
 (segment (start 151.7 77.54875) (end 157.48625 77.54875) (width 0.2) (layer "F.Cu") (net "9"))
 (segment (start 112.21625 92.63875) (end 127.30625 92.63875) (width 0.2) (layer "F.Cu") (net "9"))
 (segment (start 137.39625 60.35875) (end 133.5825 56.545) (width 0.2) (layer "F.Cu") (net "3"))
 (segment (start 133.5825 56.545) (end 108.17 56.545) (width 0.2) (layer "F.Cu") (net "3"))
 (segment (start 108.17 56.545) (end 96.71 45.085) (width 0.2) (layer "F.Cu") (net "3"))
 (segment (start 152.48625 60.35875) (end 137.39625 60.35875) (width 0.2) (layer "F.Cu") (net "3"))
 (segment (start 152.48625 90.53875) (end 152.48625 88.983116) (width 0.2) (layer "F.Cu") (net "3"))
 (segment (start 137.39625 60.35875) (end 142.276149 60.35875) (width 0.2) (layer "F.Cu") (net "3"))
 (segment (start 148.235317 84.732183) (end 147.831573 84.732183) (width 0.2) (layer "F.Cu") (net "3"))
 (segment (start 144.19625 83.73875) (end 137.39625 90.53875) (width 0.2) (layer "F.Cu") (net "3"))
 (segment (start 152.48625 88.983116) (end 148.235317 84.732183) (width 0.2) (layer "F.Cu") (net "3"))
 (segment (start 142.276149 60.35875) (end 144.19625 62.278851) (width 0.2) (layer "F.Cu") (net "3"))
 (segment (start 147.6375 76.2) (end 147.6375 78.445978) (width 0.2) (layer "F.Cu") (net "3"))
 (segment (start 144.19625 62.278851) (end 144.19625 83.73875) (width 0.2) (layer "F.Cu") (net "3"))
 (segment (start 147.6375 78.445978) (end 137.39625 88.687228) (width 0.2) (layer "F.Cu") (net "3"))
 (segment (start 137.39625 88.687228) (end 137.39625 90.53875) (width 0.2) (layer "F.Cu") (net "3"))
 (via (at 147.6375 76.2) (size 0.6) (drill 0.3) (layers "F.Cu" "B.Cu") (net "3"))
 (via (at 147.831573 84.732183) (size 0.6) (drill 0.3) (layers "F.Cu" "B.Cu") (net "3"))
 (segment (start 147.6375 76.2) (end 148.28625 76.84875) (width 0.2) (layer "B.Cu") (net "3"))
 (segment (start 148.28625 84.277506) (end 147.831573 84.732183) (width 0.2) (layer "B.Cu") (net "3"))
 (segment (start 148.28625 76.84875) (end 148.28625 84.277506) (width 0.2) (layer "B.Cu") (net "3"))
 (segment (start 111.09125 60.35875) (end 110.7375 60.7125) (width 0.2) (layer "F.Cu") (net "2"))
 (segment (start 122.30625 75.44875) (end 125.271883 72.483117) (width 0.2) (layer "F.Cu") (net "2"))
 (segment (start 109.9375 59.048629) (end 109.9375 58.878186) (width 0.2) (layer "F.Cu") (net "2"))
 (segment (start 125.271883 72.483117) (end 125.271883 67.071553) (width 0.2) (layer "F.Cu") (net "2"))
 (segment (start 110.7375 59.84863) (end 109.9375 59.048629) (width 0.2) (layer "F.Cu") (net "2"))
 (segment (start 103.446814 52.3875) (end 100.0125 52.3875) (width 0.2) (layer "F.Cu") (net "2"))
 (segment (start 110.7375 60.7125) (end 110.7375 59.84863) (width 0.2) (layer "F.Cu") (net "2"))
 (segment (start 122.30625 60.35875) (end 111.09125 60.35875) (width 0.2) (layer "F.Cu") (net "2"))
 (segment (start 109.9375 58.878186) (end 103.446814 52.3875) (width 0.2) (layer "F.Cu") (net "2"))
 (via (at 100.0125 52.3875) (size 0.6) (drill 0.3) (layers "F.Cu" "B.Cu") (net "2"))
 (via (at 125.271883 67.071553) (size 0.6) (drill 0.3) (layers "F.Cu" "B.Cu") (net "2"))
 (segment (start 125.271883 67.071553) (end 125.271883 63.324383) (width 0.2) (layer "B.Cu") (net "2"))
 (segment (start 125.18125 78.32375) (end 122.30625 75.44875) (width 0.2) (layer "B.Cu") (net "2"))
 (segment (start 96.055 48.43) (end 96.055 43.645) (width 0.2) (layer "B.Cu") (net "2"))
 (segment (start 125.18125 93.41375) (end 122.30625 90.53875) (width 0.2) (layer "B.Cu") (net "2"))
 (segment (start 125.18125 102.75375) (end 125.18125 93.41375) (width 0.2) (layer "B.Cu") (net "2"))
 (segment (start 125.271883 63.324383) (end 122.30625 60.35875) (width 0.2) (layer "B.Cu") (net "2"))
 (segment (start 96.69 49.065) (end 96.055 48.43) (width 0.2) (layer "B.Cu") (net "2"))
 (segment (start 96.055 43.645) (end 97.155 42.545) (width 0.2) (layer "B.Cu") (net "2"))
 (segment (start 97.610635 49.065) (end 96.69 49.065) (width 0.2) (layer "B.Cu") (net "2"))
 (segment (start 122.30625 90.53875) (end 125.18125 87.66375) (width 0.2) (layer "B.Cu") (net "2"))
 (segment (start 100.0125 52.3875) (end 100.0125 51.466865) (width 0.2) (layer "B.Cu") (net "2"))
 (segment (start 125.18125 87.66375) (end 125.18125 78.32375) (width 0.2) (layer "B.Cu") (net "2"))
 (segment (start 100.0125 51.466865) (end 97.610635 49.065) (width 0.2) (layer "B.Cu") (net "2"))
 (segment (start 122.30625 105.62875) (end 125.18125 102.75375) (width 0.2) (layer "B.Cu") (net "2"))
 (segment (start 142.39625 62.45875) (end 141.296251 63.558749) (width 0.2) (layer "F.Cu") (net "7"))
 (segment (start 96.71 55.245) (end 102.87 55.245) (width 0.2) (layer "F.Cu") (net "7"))
 (segment (start 109.9375 61.45875) (end 110.9375 62.45875) (width 0.2) (layer "F.Cu") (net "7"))
 (segment (start 112.21625 62.45875) (end 127.30625 62.45875) (width 0.2) (layer "F.Cu") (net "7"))
 (segment (start 141.296251 63.558749) (end 141.296251 76.448751) (width 0.2) (layer "F.Cu") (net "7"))
 (segment (start 102.87 55.245) (end 103.77 56.145) (width 0.2) (layer "F.Cu") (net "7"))
 (segment (start 127.30625 62.45875) (end 142.39625 62.45875) (width 0.2) (layer "F.Cu") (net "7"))
 (segment (start 103.77 56.145) (end 105.9025 56.145) (width 0.2) (layer "F.Cu") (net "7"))
 (segment (start 105.9025 56.145) (end 109.9375 60.180001) (width 0.2) (layer "F.Cu") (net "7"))
 (segment (start 110.9375 62.45875) (end 112.21625 62.45875) (width 0.2) (layer "F.Cu") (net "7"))
 (segment (start 141.296251 76.448751) (end 142.39625 77.54875) (width 0.2) (layer "F.Cu") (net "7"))
 (segment (start 109.9375 60.180001) (end 109.9375 61.45875) (width 0.2) (layer "F.Cu") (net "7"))
 (segment (start 141.47125 93.56375) (end 141.47125 99.573851) (width 0.2) (layer "F.Cu") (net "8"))
 (segment (start 136.816351 107.02875) (end 141.69625 107.02875) (width 0.2) (layer "F.Cu") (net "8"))
 (segment (start 110.674828 54.374119) (end 111.545709 55.245) (width 0.2) (layer "F.Cu") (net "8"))
 (segment (start 142.39625 92.63875) (end 141.47125 93.56375) (width 0.2) (layer "F.Cu") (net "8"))
 (segment (start 135.99625 105.048851) (end 135.99625 106.208649) (width 0.2) (layer "F.Cu") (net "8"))
 (segment (start 141.47125 93.56375) (end 135.03625 93.56375) (width 0.2) (layer "F.Cu") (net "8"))
 (segment (start 141.47125 99.573851) (end 135.99625 105.048851) (width 0.2) (layer "F.Cu") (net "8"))
 (segment (start 135.03625 93.56375) (end 133.35 95.25) (width 0.2) (layer "F.Cu") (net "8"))
 (segment (start 135.99625 106.208649) (end 136.816351 107.02875) (width 0.2) (layer "F.Cu") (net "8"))
 (segment (start 141.69625 107.02875) (end 142.39625 107.72875) (width 0.2) (layer "F.Cu") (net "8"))
 (segment (start 112.21625 77.54875) (end 127.30625 77.54875) (width 0.2) (layer "F.Cu") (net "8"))
 (segment (start 111.545709 55.245) (end 112.875 55.245) (width 0.2) (layer "F.Cu") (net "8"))
 (via (at 110.674828 54.374119) (size 0.6) (drill 0.3) (layers "F.Cu" "B.Cu") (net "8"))
 (via (at 133.35 95.25) (size 0.6) (drill 0.3) (layers "F.Cu" "B.Cu") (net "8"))
 (segment (start 133.35 95.25) (end 129.10625 91.00625) (width 0.2) (layer "B.Cu") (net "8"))
 (segment (start 129.10625 91.00625) (end 129.10625 79.34875) (width 0.2) (layer "B.Cu") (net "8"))
 (segment (start 112.21625 77.54875) (end 110.674828 76.007328) (width 0.2) (layer "B.Cu") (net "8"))
 (segment (start 110.674828 76.007328) (end 110.674828 54.374119) (width 0.2) (layer "B.Cu") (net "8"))
 (segment (start 129.10625 79.34875) (end 127.30625 77.54875) (width 0.2) (layer "B.Cu") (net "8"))
 (segment (start 152.48625 105.62875) (end 137.39625 105.62875) (width 0.2) (layer "F.Cu") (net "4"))
 (segment (start 140.27125 78.32375) (end 140.27125 102.75375) (width 0.2) (layer "B.Cu") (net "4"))
 (segment (start 111.295 54.789365) (end 111.616802 54.467563) (width 0.2) (layer "B.Cu") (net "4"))
 (segment (start 118.10625 60.957011) (end 113.172437 56.023198) (width 0.2) (layer "B.Cu") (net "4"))
 (segment (start 111.616802 54.467563) (end 104.774239 47.625) (width 0.2) (layer "B.Cu") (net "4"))
 (segment (start 140.27125 102.75375) (end 137.39625 105.62875) (width 0.2) (layer "B.Cu") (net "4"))
 (segment (start 104.774239 47.625) (end 97.155 47.625) (width 0.2) (layer "B.Cu") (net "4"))
 (segment (start 126.757772 75.44875) (end 118.10625 66.797228) (width 0.2) (layer "B.Cu") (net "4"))
 (segment (start 137.39625 75.44875) (end 152.48625 75.44875) (width 0.2) (layer "B.Cu") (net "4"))
 (segment (start 118.10625 66.797228) (end 118.10625 60.957011) (width 0.2) (layer "B.Cu") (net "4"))
 (segment (start 113.172437 56.023198) (end 112.850635 56.345) (width 0.2) (layer "B.Cu") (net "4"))
 (segment (start 111.939365 56.345) (end 111.295 55.700635) (width 0.2) (layer "B.Cu") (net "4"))
 (segment (start 137.39625 75.44875) (end 140.27125 78.32375) (width 0.2) (layer "B.Cu") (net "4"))
 (segment (start 111.295 55.700635) (end 111.295 54.789365) (width 0.2) (layer "B.Cu") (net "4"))
 (segment (start 137.39625 75.44875) (end 126.757772 75.44875) (width 0.2) (layer "B.Cu") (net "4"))
 (segment (start 112.850635 56.345) (end 111.939365 56.345) (width 0.2) (layer "B.Cu") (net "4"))
 (segment (start 108.61625 59.778851) (end 108.61625 60.938649) (width 0.2) (layer "B.Cu") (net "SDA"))
 (segment (start 95.255 55.679821) (end 95.255 39.705) (width 0.2) (layer "B.Cu") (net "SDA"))
 (segment (start 111.939365 41.105) (end 112.5425 41.105) (width 0.2) (layer "B.Cu") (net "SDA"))
 (segment (start 107.796149 61.75875) (end 101.333929 61.75875) (width 0.2) (layer "B.Cu") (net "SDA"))
 (segment (start 97.155 50.378529) (end 105.735221 58.95875) (width 0.2) (layer "B.Cu") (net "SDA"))
 (segment (start 97.155 50.165) (end 97.155 50.378529) (width 0.2) (layer "B.Cu") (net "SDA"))
 (segment (start 96.055 38.905) (end 109.739365 38.905) (width 0.2) (layer "B.Cu") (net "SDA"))
 (segment (start 109.739365 38.905) (end 111.939365 41.105) (width 0.2) (layer "B.Cu") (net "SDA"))
 (segment (start 105.735221 58.95875) (end 107.796149 58.95875) (width 0.2) (layer "B.Cu") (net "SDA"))
 (segment (start 101.333929 61.75875) (end 95.255 55.679821) (width 0.2) (layer "B.Cu") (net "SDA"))
 (segment (start 95.255 39.705) (end 96.055 38.905) (width 0.2) (layer "B.Cu") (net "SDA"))
 (segment (start 112.5425 41.105) (end 119.0625 47.625) (width 0.2) (layer "B.Cu") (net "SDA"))
 (segment (start 108.61625 60.938649) (end 107.796149 61.75875) (width 0.2) (layer "B.Cu") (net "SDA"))
 (segment (start 107.796149 58.95875) (end 108.61625 59.778851) (width 0.2) (layer "B.Cu") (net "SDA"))
 (segment (start 122.886149 61.75875) (end 123.825 60.819899) (width 0.2) (layer "F.Cu") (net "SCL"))
 (segment (start 110.734144 61.689707) (end 111.485202 60.938649) (width 0.2) (layer "F.Cu") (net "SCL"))
 (segment (start 96.71 52.705) (end 96.9925 52.9875) (width 0.2) (layer "F.Cu") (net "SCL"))
 (segment (start 111.485202 60.938649) (end 120.90625 60.938649) (width 0.2) (layer "F.Cu") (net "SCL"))
 (segment (start 109.5375 59.043872) (end 109.5375 59.214315) (width 0.2) (layer "F.Cu") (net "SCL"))
 (segment (start 96.9925 52.9875) (end 103.481128 52.9875) (width 0.2) (layer "F.Cu") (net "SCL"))
 (segment (start 123.825 60.819899) (end 123.825 57.15) (width 0.2) (layer "F.Cu") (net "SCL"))
 (segment (start 110.3375 61.1125) (end 110.511351 61.286351) (width 0.2) (layer "F.Cu") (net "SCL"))
 (segment (start 103.481128 52.9875) (end 109.5375 59.043872) (width 0.2) (layer "F.Cu") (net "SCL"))
 (segment (start 110.511351 61.286351) (end 110.511351 61.466915) (width 0.2) (layer "F.Cu") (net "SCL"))
 (segment (start 109.5375 59.214315) (end 110.3375 60.014316) (width 0.2) (layer "F.Cu") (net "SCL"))
 (segment (start 120.90625 60.938649) (end 121.726351 61.75875) (width 0.2) (layer "F.Cu") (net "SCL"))
 (segment (start 110.511351 61.466915) (end 110.734144 61.689707) (width 0.2) (layer "F.Cu") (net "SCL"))
 (segment (start 110.3375 60.014316) (end 110.3375 61.1125) (width 0.2) (layer "F.Cu") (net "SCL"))
 (segment (start 121.726351 61.75875) (end 122.886149 61.75875) (width 0.2) (layer "F.Cu") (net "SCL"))
 (via (at 123.825 57.15) (size 0.6) (drill 0.3) (layers "F.Cu" "B.Cu") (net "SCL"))
 (segment (start 123.825 57.15) (end 123.825 54.9275) (width 0.2) (layer "B.Cu") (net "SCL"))
 (segment (start 123.825 54.9275) (end 119.0625 50.165) (width 0.2) (layer "B.Cu") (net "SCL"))
 (segment (start 119.0625 55.245) (end 113.495 49.6775) (width 0.2) (layer "B.Cu") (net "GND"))
 (segment (start 113.495 43.645) (end 112.395 42.545) (width 0.2) (layer "B.Cu") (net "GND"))
 (segment (start 113.495 49.6775) (end 113.495 43.645) (width 0.2) (layer "B.Cu") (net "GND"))
 (segment (start 123.225 56.8675) (end 123.225 57.398529) (width 0.2) (layer "B.Cu") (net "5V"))
 (segment (start 123.225 57.398529) (end 123.576471 57.75) (width 0.2) (layer "B.Cu") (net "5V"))
 (segment (start 124.425 57.398529) (end 124.425 50.90363) (width 0.2) (layer "B.Cu") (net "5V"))
 (segment (start 119.0625 52.705) (end 123.225 56.8675) (width 0.2) (layer "B.Cu") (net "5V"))
 (segment (start 124.425 50.90363) (end 113.52637 40.005) (width 0.2) (layer "B.Cu") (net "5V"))
 (segment (start 123.576471 57.75) (end 124.073529 57.75) (width 0.2) (layer "B.Cu") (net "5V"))
 (segment (start 124.073529 57.75) (end 124.425 57.398529) (width 0.2) (layer "B.Cu") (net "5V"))
 (segment (start 113.52637 40.005) (end 112.395 40.005) (width 0.2) (layer "B.Cu") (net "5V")))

